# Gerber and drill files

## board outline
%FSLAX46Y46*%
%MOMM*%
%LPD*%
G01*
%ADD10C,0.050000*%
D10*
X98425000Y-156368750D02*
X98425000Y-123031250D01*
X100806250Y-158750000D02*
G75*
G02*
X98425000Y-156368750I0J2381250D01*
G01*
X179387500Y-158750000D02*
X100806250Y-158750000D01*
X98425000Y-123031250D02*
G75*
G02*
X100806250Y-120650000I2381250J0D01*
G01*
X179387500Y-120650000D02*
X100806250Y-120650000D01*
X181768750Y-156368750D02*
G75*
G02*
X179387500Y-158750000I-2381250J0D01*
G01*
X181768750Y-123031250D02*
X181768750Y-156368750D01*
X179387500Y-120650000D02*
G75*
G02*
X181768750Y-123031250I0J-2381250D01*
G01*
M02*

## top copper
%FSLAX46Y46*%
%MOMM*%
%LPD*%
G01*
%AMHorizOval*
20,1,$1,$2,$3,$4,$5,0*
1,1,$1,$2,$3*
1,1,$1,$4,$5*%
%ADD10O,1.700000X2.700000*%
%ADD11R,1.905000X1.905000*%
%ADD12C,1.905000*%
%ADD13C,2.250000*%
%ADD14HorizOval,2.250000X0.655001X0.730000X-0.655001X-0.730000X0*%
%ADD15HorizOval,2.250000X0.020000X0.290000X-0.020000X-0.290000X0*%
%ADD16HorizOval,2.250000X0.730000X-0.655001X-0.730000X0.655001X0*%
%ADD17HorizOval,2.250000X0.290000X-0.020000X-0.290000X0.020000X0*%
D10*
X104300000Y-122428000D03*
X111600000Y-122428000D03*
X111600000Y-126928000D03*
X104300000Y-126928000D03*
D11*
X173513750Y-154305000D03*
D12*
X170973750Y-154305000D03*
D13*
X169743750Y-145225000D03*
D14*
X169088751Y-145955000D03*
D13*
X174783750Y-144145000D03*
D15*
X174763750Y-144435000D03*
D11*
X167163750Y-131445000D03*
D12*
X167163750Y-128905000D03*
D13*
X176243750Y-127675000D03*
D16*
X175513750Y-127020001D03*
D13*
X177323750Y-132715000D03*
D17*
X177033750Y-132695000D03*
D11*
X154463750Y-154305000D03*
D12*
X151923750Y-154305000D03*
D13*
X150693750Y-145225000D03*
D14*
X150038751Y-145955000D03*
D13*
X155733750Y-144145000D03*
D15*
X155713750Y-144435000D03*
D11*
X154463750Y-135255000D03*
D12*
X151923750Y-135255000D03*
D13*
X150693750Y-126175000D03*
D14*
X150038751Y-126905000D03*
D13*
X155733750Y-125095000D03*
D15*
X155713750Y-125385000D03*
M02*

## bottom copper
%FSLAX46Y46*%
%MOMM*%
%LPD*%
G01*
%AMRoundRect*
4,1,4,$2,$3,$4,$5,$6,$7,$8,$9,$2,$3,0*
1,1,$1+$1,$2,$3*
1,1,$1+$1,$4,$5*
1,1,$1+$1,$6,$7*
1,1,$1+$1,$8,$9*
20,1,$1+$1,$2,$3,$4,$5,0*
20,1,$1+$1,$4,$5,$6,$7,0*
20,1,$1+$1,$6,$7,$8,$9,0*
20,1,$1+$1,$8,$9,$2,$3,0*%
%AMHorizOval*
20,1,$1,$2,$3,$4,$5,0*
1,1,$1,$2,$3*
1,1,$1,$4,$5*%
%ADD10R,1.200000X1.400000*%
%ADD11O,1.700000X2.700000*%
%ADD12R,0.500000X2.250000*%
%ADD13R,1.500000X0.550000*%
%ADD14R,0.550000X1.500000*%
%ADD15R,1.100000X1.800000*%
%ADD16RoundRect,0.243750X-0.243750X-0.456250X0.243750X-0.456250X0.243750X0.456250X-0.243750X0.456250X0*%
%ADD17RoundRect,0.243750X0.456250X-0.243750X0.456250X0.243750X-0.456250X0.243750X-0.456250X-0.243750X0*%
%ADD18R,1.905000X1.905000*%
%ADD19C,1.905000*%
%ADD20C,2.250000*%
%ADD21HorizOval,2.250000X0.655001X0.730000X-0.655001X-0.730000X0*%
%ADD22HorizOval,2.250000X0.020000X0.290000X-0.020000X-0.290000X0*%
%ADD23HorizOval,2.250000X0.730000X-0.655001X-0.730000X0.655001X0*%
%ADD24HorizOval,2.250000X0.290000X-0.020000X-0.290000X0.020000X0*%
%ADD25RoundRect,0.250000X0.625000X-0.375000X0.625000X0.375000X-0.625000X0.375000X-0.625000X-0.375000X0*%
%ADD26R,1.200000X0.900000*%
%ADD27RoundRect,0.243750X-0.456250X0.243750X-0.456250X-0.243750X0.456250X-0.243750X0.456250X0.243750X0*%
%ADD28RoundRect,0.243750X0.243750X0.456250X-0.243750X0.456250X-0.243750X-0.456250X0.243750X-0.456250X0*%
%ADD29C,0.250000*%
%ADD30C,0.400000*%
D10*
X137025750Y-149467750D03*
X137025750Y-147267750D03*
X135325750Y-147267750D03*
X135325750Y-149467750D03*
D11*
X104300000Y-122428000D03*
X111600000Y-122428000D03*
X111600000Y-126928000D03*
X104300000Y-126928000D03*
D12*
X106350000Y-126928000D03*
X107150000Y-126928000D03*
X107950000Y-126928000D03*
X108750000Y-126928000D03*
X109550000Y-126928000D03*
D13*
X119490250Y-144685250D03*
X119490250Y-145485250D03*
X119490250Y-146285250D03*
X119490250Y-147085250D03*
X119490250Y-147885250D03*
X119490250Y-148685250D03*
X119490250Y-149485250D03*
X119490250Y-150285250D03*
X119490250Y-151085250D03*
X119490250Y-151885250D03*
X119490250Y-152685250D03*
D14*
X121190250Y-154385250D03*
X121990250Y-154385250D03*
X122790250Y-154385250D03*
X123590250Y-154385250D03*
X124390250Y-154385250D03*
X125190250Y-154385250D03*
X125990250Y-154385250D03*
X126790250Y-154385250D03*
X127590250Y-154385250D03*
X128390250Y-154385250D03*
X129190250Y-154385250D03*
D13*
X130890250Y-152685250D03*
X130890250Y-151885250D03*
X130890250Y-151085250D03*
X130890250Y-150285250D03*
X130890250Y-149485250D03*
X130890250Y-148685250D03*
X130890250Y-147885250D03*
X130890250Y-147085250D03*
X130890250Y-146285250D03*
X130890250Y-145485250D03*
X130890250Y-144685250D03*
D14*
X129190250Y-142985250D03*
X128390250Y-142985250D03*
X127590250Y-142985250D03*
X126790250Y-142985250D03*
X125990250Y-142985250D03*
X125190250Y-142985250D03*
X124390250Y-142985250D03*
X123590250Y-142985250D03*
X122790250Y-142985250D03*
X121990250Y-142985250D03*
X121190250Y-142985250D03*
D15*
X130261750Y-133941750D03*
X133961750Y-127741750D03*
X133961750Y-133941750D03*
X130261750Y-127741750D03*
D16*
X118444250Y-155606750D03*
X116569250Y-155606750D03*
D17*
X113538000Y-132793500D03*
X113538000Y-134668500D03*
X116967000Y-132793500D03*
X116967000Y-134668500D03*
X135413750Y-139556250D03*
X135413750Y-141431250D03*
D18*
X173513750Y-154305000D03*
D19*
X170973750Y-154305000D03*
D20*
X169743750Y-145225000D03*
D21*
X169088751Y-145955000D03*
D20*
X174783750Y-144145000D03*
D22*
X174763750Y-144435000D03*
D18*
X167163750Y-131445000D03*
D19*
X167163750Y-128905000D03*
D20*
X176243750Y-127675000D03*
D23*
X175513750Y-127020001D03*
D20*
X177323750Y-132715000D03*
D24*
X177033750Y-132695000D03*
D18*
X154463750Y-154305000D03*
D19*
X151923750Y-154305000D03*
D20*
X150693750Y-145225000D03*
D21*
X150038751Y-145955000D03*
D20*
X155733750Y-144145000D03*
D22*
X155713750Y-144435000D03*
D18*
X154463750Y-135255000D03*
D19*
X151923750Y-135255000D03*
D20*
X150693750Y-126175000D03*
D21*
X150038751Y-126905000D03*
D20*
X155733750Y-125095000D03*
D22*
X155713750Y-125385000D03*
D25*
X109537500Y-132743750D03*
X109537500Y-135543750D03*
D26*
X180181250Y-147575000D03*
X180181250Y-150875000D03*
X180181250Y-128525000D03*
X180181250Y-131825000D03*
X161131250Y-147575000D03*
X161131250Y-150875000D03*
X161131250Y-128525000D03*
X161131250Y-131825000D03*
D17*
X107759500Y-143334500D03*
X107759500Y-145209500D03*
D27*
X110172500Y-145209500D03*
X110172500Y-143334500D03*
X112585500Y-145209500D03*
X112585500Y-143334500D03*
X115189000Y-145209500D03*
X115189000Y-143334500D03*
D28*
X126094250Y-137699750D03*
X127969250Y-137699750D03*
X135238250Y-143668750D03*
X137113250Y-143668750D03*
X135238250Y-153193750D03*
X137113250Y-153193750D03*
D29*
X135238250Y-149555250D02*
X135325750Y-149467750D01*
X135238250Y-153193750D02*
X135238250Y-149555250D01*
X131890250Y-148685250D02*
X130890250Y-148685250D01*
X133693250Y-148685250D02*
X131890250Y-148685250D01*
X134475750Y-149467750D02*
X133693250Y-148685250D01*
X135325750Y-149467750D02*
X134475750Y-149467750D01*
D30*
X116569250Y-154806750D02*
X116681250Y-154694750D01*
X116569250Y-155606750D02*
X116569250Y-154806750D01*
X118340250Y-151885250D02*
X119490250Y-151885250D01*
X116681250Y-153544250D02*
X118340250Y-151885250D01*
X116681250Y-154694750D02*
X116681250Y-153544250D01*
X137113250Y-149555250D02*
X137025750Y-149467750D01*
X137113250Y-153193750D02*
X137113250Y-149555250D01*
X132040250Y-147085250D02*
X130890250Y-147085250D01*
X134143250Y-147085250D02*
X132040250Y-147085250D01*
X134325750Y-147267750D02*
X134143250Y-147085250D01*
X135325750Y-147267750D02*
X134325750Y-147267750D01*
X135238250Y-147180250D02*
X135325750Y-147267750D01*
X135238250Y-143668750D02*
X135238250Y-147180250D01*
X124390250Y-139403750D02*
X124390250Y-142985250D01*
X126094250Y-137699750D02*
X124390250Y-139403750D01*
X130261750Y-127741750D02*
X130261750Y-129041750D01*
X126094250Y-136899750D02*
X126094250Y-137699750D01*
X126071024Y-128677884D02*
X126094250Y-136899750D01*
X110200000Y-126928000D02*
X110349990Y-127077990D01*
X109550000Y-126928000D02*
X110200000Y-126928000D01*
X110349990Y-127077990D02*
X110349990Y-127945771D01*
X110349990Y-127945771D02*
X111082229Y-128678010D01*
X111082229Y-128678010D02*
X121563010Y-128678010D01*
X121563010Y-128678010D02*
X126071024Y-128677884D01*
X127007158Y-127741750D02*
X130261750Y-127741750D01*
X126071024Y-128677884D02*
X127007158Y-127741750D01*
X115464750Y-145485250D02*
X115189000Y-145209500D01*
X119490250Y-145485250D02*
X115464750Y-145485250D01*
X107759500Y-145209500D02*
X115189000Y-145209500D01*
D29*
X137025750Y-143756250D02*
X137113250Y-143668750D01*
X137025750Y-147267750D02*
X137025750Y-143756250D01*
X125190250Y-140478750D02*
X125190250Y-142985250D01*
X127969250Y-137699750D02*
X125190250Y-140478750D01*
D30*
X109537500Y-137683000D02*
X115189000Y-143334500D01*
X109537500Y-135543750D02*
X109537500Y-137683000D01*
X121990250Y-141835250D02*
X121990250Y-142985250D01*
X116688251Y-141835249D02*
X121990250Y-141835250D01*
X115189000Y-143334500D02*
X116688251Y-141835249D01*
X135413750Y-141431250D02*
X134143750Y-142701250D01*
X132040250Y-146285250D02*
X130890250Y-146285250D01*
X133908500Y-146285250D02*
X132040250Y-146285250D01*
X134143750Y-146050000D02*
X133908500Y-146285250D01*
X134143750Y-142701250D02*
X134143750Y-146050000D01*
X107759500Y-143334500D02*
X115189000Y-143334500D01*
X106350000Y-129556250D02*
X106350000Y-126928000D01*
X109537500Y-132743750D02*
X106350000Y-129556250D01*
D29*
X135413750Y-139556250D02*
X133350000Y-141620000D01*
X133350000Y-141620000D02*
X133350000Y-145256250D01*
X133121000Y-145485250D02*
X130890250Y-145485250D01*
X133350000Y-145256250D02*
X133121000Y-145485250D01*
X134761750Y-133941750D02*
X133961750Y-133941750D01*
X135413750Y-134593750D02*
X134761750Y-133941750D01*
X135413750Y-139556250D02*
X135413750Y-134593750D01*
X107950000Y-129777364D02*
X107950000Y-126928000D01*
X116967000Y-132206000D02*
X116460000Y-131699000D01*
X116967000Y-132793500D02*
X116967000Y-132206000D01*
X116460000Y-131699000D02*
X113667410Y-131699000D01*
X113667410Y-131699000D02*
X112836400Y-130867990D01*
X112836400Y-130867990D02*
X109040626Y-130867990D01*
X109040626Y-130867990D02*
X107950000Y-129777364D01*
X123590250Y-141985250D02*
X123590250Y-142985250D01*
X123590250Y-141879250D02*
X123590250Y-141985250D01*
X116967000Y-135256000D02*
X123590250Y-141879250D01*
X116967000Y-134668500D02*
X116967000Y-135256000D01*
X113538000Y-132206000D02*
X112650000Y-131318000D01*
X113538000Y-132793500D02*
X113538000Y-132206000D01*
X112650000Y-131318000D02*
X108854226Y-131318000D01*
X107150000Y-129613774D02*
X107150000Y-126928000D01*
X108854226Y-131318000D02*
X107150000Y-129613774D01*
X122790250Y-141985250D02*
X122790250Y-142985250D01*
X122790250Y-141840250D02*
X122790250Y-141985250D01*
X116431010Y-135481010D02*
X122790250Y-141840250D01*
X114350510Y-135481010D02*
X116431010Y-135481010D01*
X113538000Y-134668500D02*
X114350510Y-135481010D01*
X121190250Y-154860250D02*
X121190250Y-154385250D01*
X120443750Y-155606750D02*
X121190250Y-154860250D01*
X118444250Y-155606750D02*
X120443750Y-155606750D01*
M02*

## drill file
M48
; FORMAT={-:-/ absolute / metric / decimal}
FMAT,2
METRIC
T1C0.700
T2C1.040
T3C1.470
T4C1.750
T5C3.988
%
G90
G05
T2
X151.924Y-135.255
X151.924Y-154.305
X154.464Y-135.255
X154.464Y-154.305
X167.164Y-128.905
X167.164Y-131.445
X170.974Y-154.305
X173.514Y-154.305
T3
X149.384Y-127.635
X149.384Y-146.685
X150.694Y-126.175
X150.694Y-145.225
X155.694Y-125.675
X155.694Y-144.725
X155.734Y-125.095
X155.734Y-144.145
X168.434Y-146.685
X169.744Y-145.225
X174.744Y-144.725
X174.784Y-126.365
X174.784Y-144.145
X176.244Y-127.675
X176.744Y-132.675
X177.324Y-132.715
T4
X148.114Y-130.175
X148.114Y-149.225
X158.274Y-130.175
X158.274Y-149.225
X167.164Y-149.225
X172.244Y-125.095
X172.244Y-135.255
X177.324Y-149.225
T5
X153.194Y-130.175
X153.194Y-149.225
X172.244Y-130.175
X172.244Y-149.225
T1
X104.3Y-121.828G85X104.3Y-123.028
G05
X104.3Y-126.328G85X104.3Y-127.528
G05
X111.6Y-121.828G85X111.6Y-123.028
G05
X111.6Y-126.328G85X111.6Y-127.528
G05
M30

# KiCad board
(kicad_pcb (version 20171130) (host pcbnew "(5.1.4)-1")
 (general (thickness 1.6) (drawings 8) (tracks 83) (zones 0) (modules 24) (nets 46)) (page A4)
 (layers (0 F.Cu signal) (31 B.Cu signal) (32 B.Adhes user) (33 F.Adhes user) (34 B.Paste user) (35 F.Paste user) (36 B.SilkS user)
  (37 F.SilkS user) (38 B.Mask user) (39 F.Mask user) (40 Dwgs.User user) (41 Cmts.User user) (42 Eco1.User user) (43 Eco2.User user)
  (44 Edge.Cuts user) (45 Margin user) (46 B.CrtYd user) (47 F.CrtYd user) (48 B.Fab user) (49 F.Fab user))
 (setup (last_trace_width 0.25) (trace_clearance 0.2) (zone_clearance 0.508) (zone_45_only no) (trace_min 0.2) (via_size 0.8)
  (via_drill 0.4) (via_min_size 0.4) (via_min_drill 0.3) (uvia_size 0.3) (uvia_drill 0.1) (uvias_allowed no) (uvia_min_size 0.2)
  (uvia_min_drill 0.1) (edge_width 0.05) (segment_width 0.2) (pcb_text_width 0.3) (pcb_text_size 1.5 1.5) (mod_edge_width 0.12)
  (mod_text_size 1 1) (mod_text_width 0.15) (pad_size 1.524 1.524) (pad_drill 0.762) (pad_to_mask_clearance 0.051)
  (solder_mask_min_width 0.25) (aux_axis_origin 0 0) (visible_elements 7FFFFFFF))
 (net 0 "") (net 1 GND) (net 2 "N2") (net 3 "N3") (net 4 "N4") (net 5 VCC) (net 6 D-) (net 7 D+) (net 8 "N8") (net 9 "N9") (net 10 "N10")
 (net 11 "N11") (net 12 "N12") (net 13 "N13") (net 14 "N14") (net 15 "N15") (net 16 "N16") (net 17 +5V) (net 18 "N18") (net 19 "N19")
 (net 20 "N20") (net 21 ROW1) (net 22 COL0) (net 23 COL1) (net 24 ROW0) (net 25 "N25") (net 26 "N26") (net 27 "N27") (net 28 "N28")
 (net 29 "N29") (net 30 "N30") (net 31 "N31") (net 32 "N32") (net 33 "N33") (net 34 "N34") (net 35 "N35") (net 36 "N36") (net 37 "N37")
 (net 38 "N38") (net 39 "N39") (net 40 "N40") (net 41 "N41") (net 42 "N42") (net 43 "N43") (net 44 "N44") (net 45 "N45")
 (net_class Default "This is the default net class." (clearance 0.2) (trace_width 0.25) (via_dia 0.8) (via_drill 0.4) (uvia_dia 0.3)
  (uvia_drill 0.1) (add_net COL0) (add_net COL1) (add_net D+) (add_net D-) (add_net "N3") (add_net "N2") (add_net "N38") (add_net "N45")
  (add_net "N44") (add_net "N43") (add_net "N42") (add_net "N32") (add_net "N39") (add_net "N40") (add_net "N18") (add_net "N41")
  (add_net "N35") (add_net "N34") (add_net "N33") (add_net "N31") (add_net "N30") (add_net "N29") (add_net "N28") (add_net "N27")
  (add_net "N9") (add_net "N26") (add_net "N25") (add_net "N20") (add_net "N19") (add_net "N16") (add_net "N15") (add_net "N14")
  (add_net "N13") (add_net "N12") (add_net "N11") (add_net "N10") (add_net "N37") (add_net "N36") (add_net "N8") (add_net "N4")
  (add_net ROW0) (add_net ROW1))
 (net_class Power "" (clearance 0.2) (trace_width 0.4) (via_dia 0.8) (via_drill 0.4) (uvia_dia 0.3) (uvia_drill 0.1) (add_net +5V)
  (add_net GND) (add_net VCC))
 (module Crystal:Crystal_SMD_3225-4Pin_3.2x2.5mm (layer B.Cu) (at 136.17575 148.36775 90)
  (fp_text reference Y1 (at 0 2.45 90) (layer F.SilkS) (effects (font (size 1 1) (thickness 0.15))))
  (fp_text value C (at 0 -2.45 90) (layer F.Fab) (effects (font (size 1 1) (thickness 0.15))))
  (pad 4 smd rect (at -1.1 0.85 90) (size 1.4 1.2) (layers B.Cu B.Paste B.Mask) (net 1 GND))
  (pad 3 smd rect (at 1.1 0.85 90) (size 1.4 1.2) (layers B.Cu B.Paste B.Mask) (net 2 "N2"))
  (pad 2 smd rect (at 1.1 -0.85 90) (size 1.4 1.2) (layers B.Cu B.Paste B.Mask) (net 1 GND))
  (pad 1 smd rect (at -1.1 -0.85 90) (size 1.4 1.2) (layers B.Cu B.Paste B.Mask) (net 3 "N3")))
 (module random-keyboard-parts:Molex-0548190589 (layer B.Cu) (at 107.95 122.428 270)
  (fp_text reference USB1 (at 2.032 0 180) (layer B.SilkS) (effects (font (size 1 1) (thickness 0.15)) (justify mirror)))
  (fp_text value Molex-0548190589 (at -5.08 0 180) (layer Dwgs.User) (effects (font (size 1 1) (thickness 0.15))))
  (pad 6 thru_hole oval (at 0 3.65 270) (size 2.7 1.7) (drill oval 1.9 0.7) (layers *.Cu *.Mask) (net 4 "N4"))
  (pad 6 thru_hole oval (at 0 -3.65 270) (size 2.7 1.7) (drill oval 1.9 0.7) (layers *.Cu *.Mask) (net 4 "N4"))
  (pad 6 thru_hole oval (at 4.5 -3.65 270) (size 2.7 1.7) (drill oval 1.9 0.7) (layers *.Cu *.Mask) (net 4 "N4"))
  (pad 6 thru_hole oval (at 4.5 3.65 270) (size 2.7 1.7) (drill oval 1.9 0.7) (layers *.Cu *.Mask) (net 4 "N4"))
  (pad 5 smd rect (at 4.5 1.6 270) (size 2.25 0.5) (layers B.Cu B.Paste B.Mask) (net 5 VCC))
  (pad 4 smd rect (at 4.5 0.8 270) (size 2.25 0.5) (layers B.Cu B.Paste B.Mask) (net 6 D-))
  (pad 3 smd rect (at 4.5 0 270) (size 2.25 0.5) (layers B.Cu B.Paste B.Mask) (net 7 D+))
  (pad 2 smd rect (at 4.5 -0.8 270) (size 2.25 0.5) (layers B.Cu B.Paste B.Mask) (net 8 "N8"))
  (pad 1 smd rect (at 4.5 -1.6 270) (size 2.25 0.5) (layers B.Cu B.Paste B.Mask) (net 1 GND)))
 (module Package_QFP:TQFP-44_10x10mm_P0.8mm (layer B.Cu) (at 125.19025 148.68525 270)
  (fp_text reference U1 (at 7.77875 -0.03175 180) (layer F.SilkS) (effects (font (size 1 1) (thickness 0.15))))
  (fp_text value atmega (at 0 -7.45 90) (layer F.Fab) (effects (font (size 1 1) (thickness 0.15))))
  (pad 44 smd rect (at -4 5.7 180) (size 1.5 0.55) (layers B.Cu B.Paste B.Mask) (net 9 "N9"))
  (pad 43 smd rect (at -3.2 5.7 180) (size 1.5 0.55) (layers B.Cu B.Paste B.Mask) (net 1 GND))
  (pad 42 smd rect (at -2.4 5.7 180) (size 1.5 0.55) (layers B.Cu B.Paste B.Mask) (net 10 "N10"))
  (pad 41 smd rect (at -1.6 5.7 180) (size 1.5 0.55) (layers B.Cu B.Paste B.Mask) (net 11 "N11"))
  (pad 40 smd rect (at -0.8 5.7 180) (size 1.5 0.55) (layers B.Cu B.Paste B.Mask) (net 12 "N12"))
  (pad 39 smd rect (at 0 5.7 180) (size 1.5 0.55) (layers B.Cu B.Paste B.Mask) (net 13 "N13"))
  (pad 38 smd rect (at 0.8 5.7 180) (size 1.5 0.55) (layers B.Cu B.Paste B.Mask) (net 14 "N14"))
  (pad 37 smd rect (at 1.6 5.7 180) (size 1.5 0.55) (layers B.Cu B.Paste B.Mask) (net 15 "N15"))
  (pad 36 smd rect (at 2.4 5.7 180) (size 1.5 0.55) (layers B.Cu B.Paste B.Mask) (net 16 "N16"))
  (pad 35 smd rect (at 3.2 5.7 180) (size 1.5 0.55) (layers B.Cu B.Paste B.Mask) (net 1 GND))
  (pad 34 smd rect (at 4 5.7 180) (size 1.5 0.55) (layers B.Cu B.Paste B.Mask) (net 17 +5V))
  (pad 33 smd rect (at 5.7 4 270) (size 1.5 0.55) (layers B.Cu B.Paste B.Mask) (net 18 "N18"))
  (pad 32 smd rect (at 5.7 3.2 270) (size 1.5 0.55) (layers B.Cu B.Paste B.Mask) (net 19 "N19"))
  (pad 31 smd rect (at 5.7 2.4 270) (size 1.5 0.55) (layers B.Cu B.Paste B.Mask) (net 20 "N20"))
  (pad 30 smd rect (at 5.7 1.6 270) (size 1.5 0.55) (layers B.Cu B.Paste B.Mask) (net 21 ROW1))
  (pad 29 smd rect (at 5.7 0.8 270) (size 1.5 0.55) (layers B.Cu B.Paste B.Mask) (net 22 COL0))
  (pad 28 smd rect (at 5.7 0 270) (size 1.5 0.55) (layers B.Cu B.Paste B.Mask) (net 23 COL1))
  (pad 27 smd rect (at 5.7 -0.8 270) (size 1.5 0.55) (layers B.Cu B.Paste B.Mask) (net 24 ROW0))
  (pad 26 smd rect (at 5.7 -1.6 270) (size 1.5 0.55) (layers B.Cu B.Paste B.Mask) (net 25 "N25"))
  (pad 25 smd rect (at 5.7 -2.4 270) (size 1.5 0.55) (layers B.Cu B.Paste B.Mask) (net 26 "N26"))
  (pad 24 smd rect (at 5.7 -3.2 270) (size 1.5 0.55) (layers B.Cu B.Paste B.Mask) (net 9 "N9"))
  (pad 23 smd rect (at 5.7 -4 270) (size 1.5 0.55) (layers B.Cu B.Paste B.Mask) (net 1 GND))
  (pad 22 smd rect (at 4 -5.7 180) (size 1.5 0.55) (layers B.Cu B.Paste B.Mask) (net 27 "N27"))
  (pad 21 smd rect (at 3.2 -5.7 180) (size 1.5 0.55) (layers B.Cu B.Paste B.Mask) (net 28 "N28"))
  (pad 20 smd rect (at 2.4 -5.7 180) (size 1.5 0.55) (layers B.Cu B.Paste B.Mask) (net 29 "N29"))
  (pad 19 smd rect (at 1.6 -5.7 180) (size 1.5 0.55) (layers B.Cu B.Paste B.Mask) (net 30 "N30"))
  (pad 18 smd rect (at 0.8 -5.7 180) (size 1.5 0.55) (layers B.Cu B.Paste B.Mask) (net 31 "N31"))
  (pad 17 smd rect (at 0 -5.7 180) (size 1.5 0.55) (layers B.Cu B.Paste B.Mask) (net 3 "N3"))
  (pad 16 smd rect (at -0.8 -5.7 180) (size 1.5 0.55) (layers B.Cu B.Paste B.Mask) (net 2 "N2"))
  (pad 15 smd rect (at -1.6 -5.7 180) (size 1.5 0.55) (layers B.Cu B.Paste B.Mask) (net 1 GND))
  (pad 14 smd rect (at -2.4 -5.7 180) (size 1.5 0.55) (layers B.Cu B.Paste B.Mask) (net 17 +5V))
  (pad 13 smd rect (at -3.2 -5.7 180) (size 1.5 0.55) (layers B.Cu B.Paste B.Mask) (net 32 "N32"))
  (pad 12 smd rect (at -4 -5.7 180) (size 1.5 0.55) (layers B.Cu B.Paste B.Mask) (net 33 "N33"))
  (pad 11 smd rect (at -5.7 -4 270) (size 1.5 0.55) (layers B.Cu B.Paste B.Mask) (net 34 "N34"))
  (pad 10 smd rect (at -5.7 -3.2 270) (size 1.5 0.55) (layers B.Cu B.Paste B.Mask) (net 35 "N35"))
  (pad 9 smd rect (at -5.7 -2.4 270) (size 1.5 0.55) (layers B.Cu B.Paste B.Mask) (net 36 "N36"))
  (pad 8 smd rect (at -5.7 -1.6 270) (size 1.5 0.55) (layers B.Cu B.Paste B.Mask) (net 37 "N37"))
  (pad 7 smd rect (at -5.7 -0.8 270) (size 1.5 0.55) (layers B.Cu B.Paste B.Mask) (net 17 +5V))
  (pad 6 smd rect (at -5.7 0 270) (size 1.5 0.55) (layers B.Cu B.Paste B.Mask) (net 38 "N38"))
  (pad 5 smd rect (at -5.7 0.8 270) (size 1.5 0.55) (layers B.Cu B.Paste B.Mask) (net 1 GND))
  (pad 4 smd rect (at -5.7 1.6 270) (size 1.5 0.55) (layers B.Cu B.Paste B.Mask) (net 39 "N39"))
  (pad 3 smd rect (at -5.7 2.4 270) (size 1.5 0.55) (layers B.Cu B.Paste B.Mask) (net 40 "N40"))
  (pad 2 smd rect (at -5.7 3.2 270) (size 1.5 0.55) (layers B.Cu B.Paste B.Mask) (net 17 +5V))
  (pad 1 smd rect (at -5.7 4 270) (size 1.5 0.55) (layers B.Cu B.Paste B.Mask) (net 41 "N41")))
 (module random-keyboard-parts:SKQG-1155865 (layer B.Cu) (at 132.11175 130.84175 90)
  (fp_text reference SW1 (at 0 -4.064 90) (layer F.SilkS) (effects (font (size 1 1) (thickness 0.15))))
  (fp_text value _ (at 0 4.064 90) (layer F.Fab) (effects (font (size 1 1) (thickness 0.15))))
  (pad 4 smd rect (at -3.1 -1.85 90) (size 1.8 1.1) (layers B.Cu B.Paste B.Mask))
  (pad 3 smd rect (at 3.1 1.85 90) (size 1.8 1.1) (layers B.Cu B.Paste B.Mask))
  (pad 2 smd rect (at -3.1 1.85 90) (size 1.8 1.1) (layers B.Cu B.Paste B.Mask) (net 32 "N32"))
  (pad 1 smd rect (at 3.1 -1.85 90) (size 1.8 1.1) (layers B.Cu B.Paste B.Mask) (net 1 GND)))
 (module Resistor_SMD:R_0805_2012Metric (layer B.Cu) (at 117.50675 155.60675)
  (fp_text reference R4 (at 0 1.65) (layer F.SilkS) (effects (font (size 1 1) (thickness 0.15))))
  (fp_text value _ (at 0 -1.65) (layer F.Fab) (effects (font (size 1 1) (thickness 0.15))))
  (pad 2 smd roundrect (at 0.9375 0) (size 0.975 1.4) (layers B.Cu B.Paste B.Mask) (roundrect_rratio 0.25) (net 18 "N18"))
  (pad 1 smd roundrect (at -0.9375 0) (size 0.975 1.4) (layers B.Cu B.Paste B.Mask) (roundrect_rratio 0.25) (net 1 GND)))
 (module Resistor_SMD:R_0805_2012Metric (layer B.Cu) (at 113.538 133.731 90)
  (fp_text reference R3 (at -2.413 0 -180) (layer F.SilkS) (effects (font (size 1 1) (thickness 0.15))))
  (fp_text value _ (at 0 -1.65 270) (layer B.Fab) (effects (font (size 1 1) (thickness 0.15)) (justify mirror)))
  (pad 2 smd roundrect (at 0.9375 0 90) (size 0.975 1.4) (layers B.Cu B.Paste B.Mask) (roundrect_rratio 0.25) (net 6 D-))
  (pad 1 smd roundrect (at -0.9375 0 90) (size 0.975 1.4) (layers B.Cu B.Paste B.Mask) (roundrect_rratio 0.25) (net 40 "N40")))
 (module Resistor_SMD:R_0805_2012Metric (layer B.Cu) (at 116.967 133.731 90)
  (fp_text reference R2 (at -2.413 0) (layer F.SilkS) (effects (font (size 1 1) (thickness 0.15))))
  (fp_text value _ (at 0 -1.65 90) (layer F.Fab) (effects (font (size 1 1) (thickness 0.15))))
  (pad 2 smd roundrect (at 0.9375 0 90) (size 0.975 1.4) (layers B.Cu B.Paste B.Mask) (roundrect_rratio 0.25) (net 7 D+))
  (pad 1 smd roundrect (at -0.9375 0 90) (size 0.975 1.4) (layers B.Cu B.Paste B.Mask) (roundrect_rratio 0.25) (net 39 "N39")))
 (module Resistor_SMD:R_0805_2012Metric (layer B.Cu) (at 135.41375 140.49375 90)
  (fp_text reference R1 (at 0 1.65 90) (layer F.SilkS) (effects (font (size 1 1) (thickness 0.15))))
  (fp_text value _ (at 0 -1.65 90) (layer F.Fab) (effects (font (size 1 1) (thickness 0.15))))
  (pad 2 smd roundrect (at 0.9375 0 90) (size 0.975 1.4) (layers B.Cu B.Paste B.Mask) (roundrect_rratio 0.25) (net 32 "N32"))
  (pad 1 smd roundrect (at -0.9375 0 90) (size 0.975 1.4) (layers B.Cu B.Paste B.Mask) (roundrect_rratio 0.25) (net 17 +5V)))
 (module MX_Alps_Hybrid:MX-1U (layer F.Cu) (at 172.24375 149.225)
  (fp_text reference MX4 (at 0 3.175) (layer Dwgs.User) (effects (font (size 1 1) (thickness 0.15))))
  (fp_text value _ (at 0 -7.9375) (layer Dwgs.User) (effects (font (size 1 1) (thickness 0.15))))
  (pad "" np_thru_hole circle (at 5.08 0 48.0996) (size 1.75 1.75) (drill 1.75) (layers *.Cu *.Mask))
  (pad "" np_thru_hole circle (at -5.08 0 48.0996) (size 1.75 1.75) (drill 1.75) (layers *.Cu *.Mask))
  (pad 4 thru_hole rect (at 1.27 5.08) (size 1.905 1.905) (drill 1.04) (layers *.Cu B.Mask))
  (pad 3 thru_hole circle (at -1.27 5.08) (size 1.905 1.905) (drill 1.04) (layers *.Cu B.Mask))
  (pad 1 thru_hole circle (at -2.5 -4) (size 2.25 2.25) (drill 1.47) (layers *.Cu B.Mask) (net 23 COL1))
  (pad "" np_thru_hole circle (at 0 0) (size 3.9878 3.9878) (drill 3.9878) (layers *.Cu *.Mask))
  (pad 1 thru_hole oval (at -3.81 -2.54 48.0996) (size 4.211556 2.25) (drill 1.47 (offset 0.980778 0)) (layers *.Cu B.Mask) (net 23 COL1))
  (pad 2 thru_hole circle (at 2.54 -5.08) (size 2.25 2.25) (drill 1.47) (layers *.Cu B.Mask) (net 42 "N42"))
  (pad 2 thru_hole oval (at 2.5 -4.5 86.0548) (size 2.831378 2.25) (drill 1.47 (offset 0.290689 0)) (layers *.Cu B.Mask) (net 42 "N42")))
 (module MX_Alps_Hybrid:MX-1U (layer F.Cu) (at 172.24375 130.175 270)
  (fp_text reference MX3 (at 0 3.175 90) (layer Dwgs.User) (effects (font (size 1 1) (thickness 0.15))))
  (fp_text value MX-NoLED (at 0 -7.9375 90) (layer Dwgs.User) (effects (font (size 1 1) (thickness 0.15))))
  (pad "" np_thru_hole circle (at 5.08 0 318.0996) (size 1.75 1.75) (drill 1.75) (layers *.Cu *.Mask))
  (pad "" np_thru_hole circle (at -5.08 0 318.0996) (size 1.75 1.75) (drill 1.75) (layers *.Cu *.Mask))
  (pad 4 thru_hole rect (at 1.27 5.08 270) (size 1.905 1.905) (drill 1.04) (layers *.Cu B.Mask))
  (pad 3 thru_hole circle (at -1.27 5.08 270) (size 1.905 1.905) (drill 1.04) (layers *.Cu B.Mask))
  (pad 1 thru_hole circle (at -2.5 -4 270) (size 2.25 2.25) (drill 1.47) (layers *.Cu B.Mask) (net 23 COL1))
  (pad "" np_thru_hole circle (at 0 0 270) (size 3.9878 3.9878) (drill 3.9878) (layers *.Cu *.Mask))
  (pad 1 thru_hole oval (at -3.81 -2.54 318.0996) (size 4.211556 2.25) (drill 1.47 (offset 0.980778 0)) (layers *.Cu B.Mask) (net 23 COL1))
  (pad 2 thru_hole circle (at 2.54 -5.08 270) (size 2.25 2.25) (drill 1.47) (layers *.Cu B.Mask) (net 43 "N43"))
  (pad 2 thru_hole oval (at 2.5 -4.5 356.0548) (size 2.831378 2.25) (drill 1.47 (offset 0.290689 0)) (layers *.Cu B.Mask) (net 43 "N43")))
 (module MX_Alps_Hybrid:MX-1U (layer F.Cu) (at 153.19375 149.225)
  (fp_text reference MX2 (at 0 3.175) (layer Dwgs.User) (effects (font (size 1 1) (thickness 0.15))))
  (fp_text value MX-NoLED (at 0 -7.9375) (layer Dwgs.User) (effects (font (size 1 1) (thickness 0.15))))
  (pad "" np_thru_hole circle (at 5.08 0 48.0996) (size 1.75 1.75) (drill 1.75) (layers *.Cu *.Mask))
  (pad "" np_thru_hole circle (at -5.08 0 48.0996) (size 1.75 1.75) (drill 1.75) (layers *.Cu *.Mask))
  (pad 4 thru_hole rect (at 1.27 5.08) (size 1.905 1.905) (drill 1.04) (layers *.Cu B.Mask))
  (pad 3 thru_hole circle (at -1.27 5.08) (size 1.905 1.905) (drill 1.04) (layers *.Cu B.Mask))
  (pad 1 thru_hole circle (at -2.5 -4) (size 2.25 2.25) (drill 1.47) (layers *.Cu B.Mask) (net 22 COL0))
  (pad "" np_thru_hole circle (at 0 0) (size 3.9878 3.9878) (drill 3.9878) (layers *.Cu *.Mask))
  (pad 1 thru_hole oval (at -3.81 -2.54 48.0996) (size 4.211556 2.25) (drill 1.47 (offset 0.980778 0)) (layers *.Cu B.Mask) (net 22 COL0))
  (pad 2 thru_hole circle (at 2.54 -5.08) (size 2.25 2.25) (drill 1.47) (layers *.Cu B.Mask) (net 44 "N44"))
  (pad 2 thru_hole oval (at 2.5 -4.5 86.0548) (size 2.831378 2.25) (drill 1.47 (offset 0.290689 0)) (layers *.Cu B.Mask) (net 44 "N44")))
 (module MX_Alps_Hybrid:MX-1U (layer F.Cu) (at 153.19375 130.175)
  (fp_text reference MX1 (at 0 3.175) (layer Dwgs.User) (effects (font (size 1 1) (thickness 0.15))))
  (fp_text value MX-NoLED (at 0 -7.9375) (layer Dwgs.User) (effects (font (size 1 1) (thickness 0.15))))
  (pad "" np_thru_hole circle (at 5.08 0 48.0996) (size 1.75 1.75) (drill 1.75) (layers *.Cu *.Mask))
  (pad "" np_thru_hole circle (at -5.08 0 48.0996) (size 1.75 1.75) (drill 1.75) (layers *.Cu *.Mask))
  (pad 4 thru_hole rect (at 1.27 5.08) (size 1.905 1.905) (drill 1.04) (layers *.Cu B.Mask))
  (pad 3 thru_hole circle (at -1.27 5.08) (size 1.905 1.905) (drill 1.04) (layers *.Cu B.Mask))
  (pad 1 thru_hole circle (at -2.5 -4) (size 2.25 2.25) (drill 1.47) (layers *.Cu B.Mask) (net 22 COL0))
  (pad "" np_thru_hole circle (at 0 0) (size 3.9878 3.9878) (drill 3.9878) (layers *.Cu *.Mask))
  (pad 1 thru_hole oval (at -3.81 -2.54 48.0996) (size 4.211556 2.25) (drill 1.47 (offset 0.980778 0)) (layers *.Cu B.Mask) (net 22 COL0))
  (pad 2 thru_hole circle (at 2.54 -5.08) (size 2.25 2.25) (drill 1.47) (layers *.Cu B.Mask) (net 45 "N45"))
  (pad 2 thru_hole oval (at 2.5 -4.5 86.0548) (size 2.831378 2.25) (drill 1.47 (offset 0.290689 0)) (layers *.Cu B.Mask) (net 45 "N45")))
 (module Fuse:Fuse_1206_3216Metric (layer B.Cu) (at 109.5375 134.14375 90)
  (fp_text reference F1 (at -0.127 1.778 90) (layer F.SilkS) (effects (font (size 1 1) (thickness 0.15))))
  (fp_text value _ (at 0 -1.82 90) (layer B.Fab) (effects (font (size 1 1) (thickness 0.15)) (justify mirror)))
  (pad 2 smd roundrect (at 1.4 0 90) (size 1.25 1.75) (layers B.Cu B.Paste B.Mask) (roundrect_rratio 0.2) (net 5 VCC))
  (pad 1 smd roundrect (at -1.4 0 90) (size 1.25 1.75) (layers B.Cu B.Paste B.Mask) (roundrect_rratio 0.2) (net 17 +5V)))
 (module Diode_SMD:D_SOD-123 (layer B.Cu) (at 180.18125 149.225 90)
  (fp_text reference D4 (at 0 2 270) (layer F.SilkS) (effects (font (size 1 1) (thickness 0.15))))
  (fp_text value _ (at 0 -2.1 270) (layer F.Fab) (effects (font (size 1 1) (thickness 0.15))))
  (pad 2 smd rect (at 1.65 0 90) (size 0.9 1.2) (layers B.Cu B.Paste B.Mask) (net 42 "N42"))
  (pad 1 smd rect (at -1.65 0 90) (size 0.9 1.2) (layers B.Cu B.Paste B.Mask) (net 21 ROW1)))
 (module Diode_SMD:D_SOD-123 (layer B.Cu) (at 180.18125 130.175 90)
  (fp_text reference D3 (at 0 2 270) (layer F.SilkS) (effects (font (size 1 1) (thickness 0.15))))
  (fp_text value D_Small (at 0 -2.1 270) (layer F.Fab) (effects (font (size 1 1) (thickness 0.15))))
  (pad 2 smd rect (at 1.65 0 90) (size 0.9 1.2) (layers B.Cu B.Paste B.Mask) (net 43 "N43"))
  (pad 1 smd rect (at -1.65 0 90) (size 0.9 1.2) (layers B.Cu B.Paste B.Mask) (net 24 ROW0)))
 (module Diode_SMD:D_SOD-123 (layer B.Cu) (at 161.13125 149.225 90)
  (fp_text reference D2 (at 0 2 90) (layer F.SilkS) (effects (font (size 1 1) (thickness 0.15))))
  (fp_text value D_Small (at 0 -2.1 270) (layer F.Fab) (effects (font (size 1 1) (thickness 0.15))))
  (pad 2 smd rect (at 1.65 0 90) (size 0.9 1.2) (layers B.Cu B.Paste B.Mask) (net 44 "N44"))
  (pad 1 smd rect (at -1.65 0 90) (size 0.9 1.2) (layers B.Cu B.Paste B.Mask) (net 21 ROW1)))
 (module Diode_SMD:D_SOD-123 (layer B.Cu) (at 161.13125 130.175 90)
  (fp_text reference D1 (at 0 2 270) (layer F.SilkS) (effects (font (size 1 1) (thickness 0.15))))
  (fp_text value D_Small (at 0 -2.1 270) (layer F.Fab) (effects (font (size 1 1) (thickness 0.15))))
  (pad 2 smd rect (at 1.65 0 90) (size 0.9 1.2) (layers B.Cu B.Paste B.Mask) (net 45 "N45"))
  (pad 1 smd rect (at -1.65 0 90) (size 0.9 1.2) (layers B.Cu B.Paste B.Mask) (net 24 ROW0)))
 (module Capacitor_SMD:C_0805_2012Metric (layer B.Cu) (at 107.7595 144.272 90)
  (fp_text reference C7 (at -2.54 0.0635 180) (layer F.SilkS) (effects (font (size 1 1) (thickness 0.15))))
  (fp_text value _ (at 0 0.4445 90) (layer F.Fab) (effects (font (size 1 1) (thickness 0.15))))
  (pad 2 smd roundrect (at 0.9375 0 90) (size 0.975 1.4) (layers B.Cu B.Paste B.Mask) (roundrect_rratio 0.25) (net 17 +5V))
  (pad 1 smd roundrect (at -0.9375 0 90) (size 0.975 1.4) (layers B.Cu B.Paste B.Mask) (roundrect_rratio 0.25) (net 1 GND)))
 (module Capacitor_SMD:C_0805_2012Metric (layer B.Cu) (at 110.1725 144.272 270)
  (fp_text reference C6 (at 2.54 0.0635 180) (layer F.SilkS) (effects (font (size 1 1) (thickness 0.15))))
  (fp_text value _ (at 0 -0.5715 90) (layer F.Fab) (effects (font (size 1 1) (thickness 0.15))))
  (pad 2 smd roundrect (at 0.9375 0 270) (size 0.975 1.4) (layers B.Cu B.Paste B.Mask) (roundrect_rratio 0.25) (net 1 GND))
  (pad 1 smd roundrect (at -0.9375 0 270) (size 0.975 1.4) (layers B.Cu B.Paste B.Mask) (roundrect_rratio 0.25) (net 17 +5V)))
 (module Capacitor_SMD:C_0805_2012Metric (layer B.Cu) (at 112.5855 144.272 270)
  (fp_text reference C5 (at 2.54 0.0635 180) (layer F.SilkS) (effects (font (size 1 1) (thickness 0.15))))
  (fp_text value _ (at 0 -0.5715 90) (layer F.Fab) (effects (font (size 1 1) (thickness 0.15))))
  (pad 2 smd roundrect (at 0.9375 0 270) (size 0.975 1.4) (layers B.Cu B.Paste B.Mask) (roundrect_rratio 0.25) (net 1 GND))
  (pad 1 smd roundrect (at -0.9375 0 270) (size 0.975 1.4) (layers B.Cu B.Paste B.Mask) (roundrect_rratio 0.25) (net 17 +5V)))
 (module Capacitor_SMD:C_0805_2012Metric (layer B.Cu) (at 115.189 144.272 270)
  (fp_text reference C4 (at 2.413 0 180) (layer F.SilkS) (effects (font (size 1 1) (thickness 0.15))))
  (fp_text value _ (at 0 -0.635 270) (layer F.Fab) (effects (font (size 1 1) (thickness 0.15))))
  (pad 2 smd roundrect (at 0.9375 0 270) (size 0.975 1.4) (layers B.Cu B.Paste B.Mask) (roundrect_rratio 0.25) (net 1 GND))
  (pad 1 smd roundrect (at -0.9375 0 270) (size 0.975 1.4) (layers B.Cu B.Paste B.Mask) (roundrect_rratio 0.25) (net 17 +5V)))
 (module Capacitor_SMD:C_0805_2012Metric (layer B.Cu) (at 127.03175 137.69975 180)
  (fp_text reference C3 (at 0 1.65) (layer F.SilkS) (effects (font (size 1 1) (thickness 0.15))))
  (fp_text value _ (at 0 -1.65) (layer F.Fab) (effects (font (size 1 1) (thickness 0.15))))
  (pad 2 smd roundrect (at 0.9375 0 180) (size 0.975 1.4) (layers B.Cu B.Paste B.Mask) (roundrect_rratio 0.25) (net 1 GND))
  (pad 1 smd roundrect (at -0.9375 0 180) (size 0.975 1.4) (layers B.Cu B.Paste B.Mask) (roundrect_rratio 0.25) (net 38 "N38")))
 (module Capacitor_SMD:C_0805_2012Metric (layer B.Cu) (at 136.17575 143.66875 180)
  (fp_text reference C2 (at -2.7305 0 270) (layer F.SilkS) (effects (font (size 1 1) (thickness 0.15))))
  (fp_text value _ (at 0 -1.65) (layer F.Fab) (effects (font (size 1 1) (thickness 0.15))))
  (pad 2 smd roundrect (at 0.9375 0 180) (size 0.975 1.4) (layers B.Cu B.Paste B.Mask) (roundrect_rratio 0.25) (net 1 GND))
  (pad 1 smd roundrect (at -0.9375 0 180) (size 0.975 1.4) (layers B.Cu B.Paste B.Mask) (roundrect_rratio 0.25) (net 2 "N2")))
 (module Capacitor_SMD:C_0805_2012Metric (layer B.Cu) (at 136.17575 153.19375 180)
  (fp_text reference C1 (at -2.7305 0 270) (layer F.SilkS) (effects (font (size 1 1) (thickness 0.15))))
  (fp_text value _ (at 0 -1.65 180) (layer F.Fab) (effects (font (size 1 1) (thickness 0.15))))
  (pad 2 smd roundrect (at 0.9375 0 180) (size 0.975 1.4) (layers B.Cu B.Paste B.Mask) (roundrect_rratio 0.25) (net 3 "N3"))
  (pad 1 smd roundrect (at -0.9375 0 180) (size 0.975 1.4) (layers B.Cu B.Paste B.Mask) (roundrect_rratio 0.25) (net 1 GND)))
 (gr_line (start 98.425 156.36875) (end 98.425 123.03125) (layer Edge.Cuts) (width 0.05))
 (gr_arc (start 100.80625 156.36875) (end 98.425 156.36875) (angle -90) (layer Edge.Cuts) (width 0.05))
 (gr_line (start 179.3875 158.75) (end 100.80625 158.75) (layer Edge.Cuts) (width 0.05))
 (gr_arc (start 100.80625 123.03125) (end 100.80625 120.65) (angle -90) (layer Edge.Cuts) (width 0.05))
 (gr_line (start 179.3875 120.65) (end 100.80625 120.65) (layer Edge.Cuts) (width 0.05))
 (gr_arc (start 179.3875 156.36875) (end 179.3875 158.75) (angle -90) (layer Edge.Cuts) (width 0.05))
 (gr_line (start 181.76875 123.03125) (end 181.76875 156.36875) (layer Edge.Cuts) (width 0.05))
 (gr_arc (start 179.3875 123.03125) (end 181.76875 123.03125) (angle -90) (layer Edge.Cuts) (width 0.05))
 (segment (start 135.23825 149.55525) (end 135.32575 149.46775) (width 0.25) (layer B.Cu) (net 3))
 (segment (start 135.23825 153.19375) (end 135.23825 149.55525) (width 0.25) (layer B.Cu) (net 3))
 (segment (start 131.89025 148.68525) (end 130.89025 148.68525) (width 0.25) (layer B.Cu) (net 3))
 (segment (start 133.69325 148.68525) (end 131.89025 148.68525) (width 0.25) (layer B.Cu) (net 3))
 (segment (start 134.47575 149.46775) (end 133.69325 148.68525) (width 0.25) (layer B.Cu) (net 3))
 (segment (start 135.32575 149.46775) (end 134.47575 149.46775) (width 0.25) (layer B.Cu) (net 3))
 (segment (start 116.56925 154.80675) (end 116.68125 154.69475) (width 0.4) (layer B.Cu) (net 1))
 (segment (start 116.56925 155.60675) (end 116.56925 154.80675) (width 0.4) (layer B.Cu) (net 1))
 (segment (start 118.34025 151.88525) (end 119.49025 151.88525) (width 0.4) (layer B.Cu) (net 1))
 (segment (start 116.68125 153.54425) (end 118.34025 151.88525) (width 0.4) (layer B.Cu) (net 1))
 (segment (start 116.68125 154.69475) (end 116.68125 153.54425) (width 0.4) (layer B.Cu) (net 1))
 (segment (start 137.11325 149.55525) (end 137.02575 149.46775) (width 0.4) (layer B.Cu) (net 1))
 (segment (start 137.11325 153.19375) (end 137.11325 149.55525) (width 0.4) (layer B.Cu) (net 1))
 (segment (start 132.04025 147.08525) (end 130.89025 147.08525) (width 0.4) (layer B.Cu) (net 1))
 (segment (start 134.14325 147.08525) (end 132.04025 147.08525) (width 0.4) (layer B.Cu) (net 1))
 (segment (start 134.32575 147.26775) (end 134.14325 147.08525) (width 0.4) (layer B.Cu) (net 1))
 (segment (start 135.32575 147.26775) (end 134.32575 147.26775) (width 0.4) (layer B.Cu) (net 1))
 (segment (start 135.23825 147.18025) (end 135.32575 147.26775) (width 0.4) (layer B.Cu) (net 1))
 (segment (start 135.23825 143.66875) (end 135.23825 147.18025) (width 0.4) (layer B.Cu) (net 1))
 (segment (start 124.39025 139.40375) (end 124.39025 142.98525) (width 0.4) (layer B.Cu) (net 1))
 (segment (start 126.09425 137.69975) (end 124.39025 139.40375) (width 0.4) (layer B.Cu) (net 1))
 (segment (start 130.26175 127.74175) (end 130.26175 129.04175) (width 0.4) (layer B.Cu) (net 1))
 (segment (start 126.09425 136.89975) (end 126.09425 137.69975) (width 0.4) (layer B.Cu) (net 1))
 (segment (start 126.071024 128.677884) (end 126.09425 136.89975) (width 0.4) (layer B.Cu) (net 1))
 (segment (start 110.2 126.928) (end 110.34999 127.07799) (width 0.4) (layer B.Cu) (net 1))
 (segment (start 109.55 126.928) (end 110.2 126.928) (width 0.4) (layer B.Cu) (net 1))
 (segment (start 110.34999 127.07799) (end 110.34999 127.945771) (width 0.4) (layer B.Cu) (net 1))
 (segment (start 110.34999 127.945771) (end 111.082229 128.67801) (width 0.4) (layer B.Cu) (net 1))
 (segment (start 111.082229 128.67801) (end 121.56301 128.67801) (width 0.4) (layer B.Cu) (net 1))
 (segment (start 121.56301 128.67801) (end 126.071024 128.677884) (width 0.4) (layer B.Cu) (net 1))
 (segment (start 127.007158 127.74175) (end 130.26175 127.74175) (width 0.4) (layer B.Cu) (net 1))
 (segment (start 126.071024 128.677884) (end 127.007158 127.74175) (width 0.4) (layer B.Cu) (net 1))
 (segment (start 115.46475 145.48525) (end 115.189 145.2095) (width 0.4) (layer B.Cu) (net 1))
 (segment (start 119.49025 145.48525) (end 115.46475 145.48525) (width 0.4) (layer B.Cu) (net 1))
 (segment (start 107.7595 145.2095) (end 115.189 145.2095) (width 0.4) (layer B.Cu) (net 1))
 (segment (start 137.02575 143.75625) (end 137.11325 143.66875) (width 0.25) (layer B.Cu) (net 2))
 (segment (start 137.02575 147.26775) (end 137.02575 143.75625) (width 0.25) (layer B.Cu) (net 2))
 (segment (start 125.19025 140.47875) (end 125.19025 142.98525) (width 0.25) (layer B.Cu) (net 38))
 (segment (start 127.96925 137.69975) (end 125.19025 140.47875) (width 0.25) (layer B.Cu) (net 38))
 (segment (start 109.5375 137.683) (end 115.189 143.3345) (width 0.4) (layer B.Cu) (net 17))
 (segment (start 109.5375 135.54375) (end 109.5375 137.683) (width 0.4) (layer B.Cu) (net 17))
 (segment (start 121.99025 141.83525) (end 121.99025 142.98525) (width 0.4) (layer B.Cu) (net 17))
 (segment (start 116.688251 141.835249) (end 121.99025 141.83525) (width 0.4) (layer B.Cu) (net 17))
 (segment (start 115.189 143.3345) (end 116.688251 141.835249) (width 0.4) (layer B.Cu) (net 17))
 (segment (start 135.41375 141.43125) (end 134.14375 142.70125) (width 0.4) (layer B.Cu) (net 17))
 (segment (start 132.04025 146.28525) (end 130.89025 146.28525) (width 0.4) (layer B.Cu) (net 17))
 (segment (start 133.9085 146.28525) (end 132.04025 146.28525) (width 0.4) (layer B.Cu) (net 17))
 (segment (start 134.14375 146.05) (end 133.9085 146.28525) (width 0.4) (layer B.Cu) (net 17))
 (segment (start 134.14375 142.70125) (end 134.14375 146.05) (width 0.4) (layer B.Cu) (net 17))
 (segment (start 107.7595 143.3345) (end 115.189 143.3345) (width 0.4) (layer B.Cu) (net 17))
 (segment (start 106.35 129.55625) (end 106.35 126.928) (width 0.4) (layer B.Cu) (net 5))
 (segment (start 109.5375 132.74375) (end 106.35 129.55625) (width 0.4) (layer B.Cu) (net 5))
 (segment (start 135.41375 139.55625) (end 133.35 141.62) (width 0.25) (layer B.Cu) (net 32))
 (segment (start 133.35 141.62) (end 133.35 145.25625) (width 0.25) (layer B.Cu) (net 32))
 (segment (start 133.121 145.48525) (end 130.89025 145.48525) (width 0.25) (layer B.Cu) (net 32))
 (segment (start 133.35 145.25625) (end 133.121 145.48525) (width 0.25) (layer B.Cu) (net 32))
 (segment (start 134.76175 133.94175) (end 133.96175 133.94175) (width 0.25) (layer B.Cu) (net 32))
 (segment (start 135.41375 134.59375) (end 134.76175 133.94175) (width 0.25) (layer B.Cu) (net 32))
 (segment (start 135.41375 139.55625) (end 135.41375 134.59375) (width 0.25) (layer B.Cu) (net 32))
 (segment (start 107.95 129.777364) (end 107.95 126.928) (width 0.25) (layer B.Cu) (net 7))
 (segment (start 116.967 132.206) (end 116.46 131.699) (width 0.25) (layer B.Cu) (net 7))
 (segment (start 116.967 132.7935) (end 116.967 132.206) (width 0.25) (layer B.Cu) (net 7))
 (segment (start 116.46 131.699) (end 113.66741 131.699) (width 0.25) (layer B.Cu) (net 7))
 (segment (start 113.66741 131.699) (end 112.8364 130.86799) (width 0.25) (layer B.Cu) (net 7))
 (segment (start 112.8364 130.86799) (end 109.040626 130.86799) (width 0.25) (layer B.Cu) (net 7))
 (segment (start 109.040626 130.86799) (end 107.95 129.777364) (width 0.25) (layer B.Cu) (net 7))
 (segment (start 123.59025 141.98525) (end 123.59025 142.98525) (width 0.25) (layer B.Cu) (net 39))
 (segment (start 123.59025 141.87925) (end 123.59025 141.98525) (width 0.25) (layer B.Cu) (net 39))
 (segment (start 116.967 135.256) (end 123.59025 141.87925) (width 0.25) (layer B.Cu) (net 39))
 (segment (start 116.967 134.6685) (end 116.967 135.256) (width 0.25) (layer B.Cu) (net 39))
 (segment (start 113.538 132.206) (end 112.65 131.318) (width 0.25) (layer B.Cu) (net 6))
 (segment (start 113.538 132.7935) (end 113.538 132.206) (width 0.25) (layer B.Cu) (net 6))
 (segment (start 112.65 131.318) (end 108.854226 131.318) (width 0.25) (layer B.Cu) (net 6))
 (segment (start 107.15 129.613774) (end 107.15 126.928) (width 0.25) (layer B.Cu) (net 6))
 (segment (start 108.854226 131.318) (end 107.15 129.613774) (width 0.25) (layer B.Cu) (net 6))
 (segment (start 122.79025 141.98525) (end 122.79025 142.98525) (width 0.25) (layer B.Cu) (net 40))
 (segment (start 122.79025 141.84025) (end 122.79025 141.98525) (width 0.25) (layer B.Cu) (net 40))
 (segment (start 116.43101 135.48101) (end 122.79025 141.84025) (width 0.25) (layer B.Cu) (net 40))
 (segment (start 114.35051 135.48101) (end 116.43101 135.48101) (width 0.25) (layer B.Cu) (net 40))
 (segment (start 113.538 134.6685) (end 114.35051 135.48101) (width 0.25) (layer B.Cu) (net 40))
 (segment (start 121.19025 154.86025) (end 121.19025 154.38525) (width 0.25) (layer B.Cu) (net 18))
 (segment (start 120.44375 155.60675) (end 121.19025 154.86025) (width 0.25) (layer B.Cu) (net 18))
 (segment (start 118.44425 155.60675) (end 120.44375 155.60675) (width 0.25) (layer B.Cu) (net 18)))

